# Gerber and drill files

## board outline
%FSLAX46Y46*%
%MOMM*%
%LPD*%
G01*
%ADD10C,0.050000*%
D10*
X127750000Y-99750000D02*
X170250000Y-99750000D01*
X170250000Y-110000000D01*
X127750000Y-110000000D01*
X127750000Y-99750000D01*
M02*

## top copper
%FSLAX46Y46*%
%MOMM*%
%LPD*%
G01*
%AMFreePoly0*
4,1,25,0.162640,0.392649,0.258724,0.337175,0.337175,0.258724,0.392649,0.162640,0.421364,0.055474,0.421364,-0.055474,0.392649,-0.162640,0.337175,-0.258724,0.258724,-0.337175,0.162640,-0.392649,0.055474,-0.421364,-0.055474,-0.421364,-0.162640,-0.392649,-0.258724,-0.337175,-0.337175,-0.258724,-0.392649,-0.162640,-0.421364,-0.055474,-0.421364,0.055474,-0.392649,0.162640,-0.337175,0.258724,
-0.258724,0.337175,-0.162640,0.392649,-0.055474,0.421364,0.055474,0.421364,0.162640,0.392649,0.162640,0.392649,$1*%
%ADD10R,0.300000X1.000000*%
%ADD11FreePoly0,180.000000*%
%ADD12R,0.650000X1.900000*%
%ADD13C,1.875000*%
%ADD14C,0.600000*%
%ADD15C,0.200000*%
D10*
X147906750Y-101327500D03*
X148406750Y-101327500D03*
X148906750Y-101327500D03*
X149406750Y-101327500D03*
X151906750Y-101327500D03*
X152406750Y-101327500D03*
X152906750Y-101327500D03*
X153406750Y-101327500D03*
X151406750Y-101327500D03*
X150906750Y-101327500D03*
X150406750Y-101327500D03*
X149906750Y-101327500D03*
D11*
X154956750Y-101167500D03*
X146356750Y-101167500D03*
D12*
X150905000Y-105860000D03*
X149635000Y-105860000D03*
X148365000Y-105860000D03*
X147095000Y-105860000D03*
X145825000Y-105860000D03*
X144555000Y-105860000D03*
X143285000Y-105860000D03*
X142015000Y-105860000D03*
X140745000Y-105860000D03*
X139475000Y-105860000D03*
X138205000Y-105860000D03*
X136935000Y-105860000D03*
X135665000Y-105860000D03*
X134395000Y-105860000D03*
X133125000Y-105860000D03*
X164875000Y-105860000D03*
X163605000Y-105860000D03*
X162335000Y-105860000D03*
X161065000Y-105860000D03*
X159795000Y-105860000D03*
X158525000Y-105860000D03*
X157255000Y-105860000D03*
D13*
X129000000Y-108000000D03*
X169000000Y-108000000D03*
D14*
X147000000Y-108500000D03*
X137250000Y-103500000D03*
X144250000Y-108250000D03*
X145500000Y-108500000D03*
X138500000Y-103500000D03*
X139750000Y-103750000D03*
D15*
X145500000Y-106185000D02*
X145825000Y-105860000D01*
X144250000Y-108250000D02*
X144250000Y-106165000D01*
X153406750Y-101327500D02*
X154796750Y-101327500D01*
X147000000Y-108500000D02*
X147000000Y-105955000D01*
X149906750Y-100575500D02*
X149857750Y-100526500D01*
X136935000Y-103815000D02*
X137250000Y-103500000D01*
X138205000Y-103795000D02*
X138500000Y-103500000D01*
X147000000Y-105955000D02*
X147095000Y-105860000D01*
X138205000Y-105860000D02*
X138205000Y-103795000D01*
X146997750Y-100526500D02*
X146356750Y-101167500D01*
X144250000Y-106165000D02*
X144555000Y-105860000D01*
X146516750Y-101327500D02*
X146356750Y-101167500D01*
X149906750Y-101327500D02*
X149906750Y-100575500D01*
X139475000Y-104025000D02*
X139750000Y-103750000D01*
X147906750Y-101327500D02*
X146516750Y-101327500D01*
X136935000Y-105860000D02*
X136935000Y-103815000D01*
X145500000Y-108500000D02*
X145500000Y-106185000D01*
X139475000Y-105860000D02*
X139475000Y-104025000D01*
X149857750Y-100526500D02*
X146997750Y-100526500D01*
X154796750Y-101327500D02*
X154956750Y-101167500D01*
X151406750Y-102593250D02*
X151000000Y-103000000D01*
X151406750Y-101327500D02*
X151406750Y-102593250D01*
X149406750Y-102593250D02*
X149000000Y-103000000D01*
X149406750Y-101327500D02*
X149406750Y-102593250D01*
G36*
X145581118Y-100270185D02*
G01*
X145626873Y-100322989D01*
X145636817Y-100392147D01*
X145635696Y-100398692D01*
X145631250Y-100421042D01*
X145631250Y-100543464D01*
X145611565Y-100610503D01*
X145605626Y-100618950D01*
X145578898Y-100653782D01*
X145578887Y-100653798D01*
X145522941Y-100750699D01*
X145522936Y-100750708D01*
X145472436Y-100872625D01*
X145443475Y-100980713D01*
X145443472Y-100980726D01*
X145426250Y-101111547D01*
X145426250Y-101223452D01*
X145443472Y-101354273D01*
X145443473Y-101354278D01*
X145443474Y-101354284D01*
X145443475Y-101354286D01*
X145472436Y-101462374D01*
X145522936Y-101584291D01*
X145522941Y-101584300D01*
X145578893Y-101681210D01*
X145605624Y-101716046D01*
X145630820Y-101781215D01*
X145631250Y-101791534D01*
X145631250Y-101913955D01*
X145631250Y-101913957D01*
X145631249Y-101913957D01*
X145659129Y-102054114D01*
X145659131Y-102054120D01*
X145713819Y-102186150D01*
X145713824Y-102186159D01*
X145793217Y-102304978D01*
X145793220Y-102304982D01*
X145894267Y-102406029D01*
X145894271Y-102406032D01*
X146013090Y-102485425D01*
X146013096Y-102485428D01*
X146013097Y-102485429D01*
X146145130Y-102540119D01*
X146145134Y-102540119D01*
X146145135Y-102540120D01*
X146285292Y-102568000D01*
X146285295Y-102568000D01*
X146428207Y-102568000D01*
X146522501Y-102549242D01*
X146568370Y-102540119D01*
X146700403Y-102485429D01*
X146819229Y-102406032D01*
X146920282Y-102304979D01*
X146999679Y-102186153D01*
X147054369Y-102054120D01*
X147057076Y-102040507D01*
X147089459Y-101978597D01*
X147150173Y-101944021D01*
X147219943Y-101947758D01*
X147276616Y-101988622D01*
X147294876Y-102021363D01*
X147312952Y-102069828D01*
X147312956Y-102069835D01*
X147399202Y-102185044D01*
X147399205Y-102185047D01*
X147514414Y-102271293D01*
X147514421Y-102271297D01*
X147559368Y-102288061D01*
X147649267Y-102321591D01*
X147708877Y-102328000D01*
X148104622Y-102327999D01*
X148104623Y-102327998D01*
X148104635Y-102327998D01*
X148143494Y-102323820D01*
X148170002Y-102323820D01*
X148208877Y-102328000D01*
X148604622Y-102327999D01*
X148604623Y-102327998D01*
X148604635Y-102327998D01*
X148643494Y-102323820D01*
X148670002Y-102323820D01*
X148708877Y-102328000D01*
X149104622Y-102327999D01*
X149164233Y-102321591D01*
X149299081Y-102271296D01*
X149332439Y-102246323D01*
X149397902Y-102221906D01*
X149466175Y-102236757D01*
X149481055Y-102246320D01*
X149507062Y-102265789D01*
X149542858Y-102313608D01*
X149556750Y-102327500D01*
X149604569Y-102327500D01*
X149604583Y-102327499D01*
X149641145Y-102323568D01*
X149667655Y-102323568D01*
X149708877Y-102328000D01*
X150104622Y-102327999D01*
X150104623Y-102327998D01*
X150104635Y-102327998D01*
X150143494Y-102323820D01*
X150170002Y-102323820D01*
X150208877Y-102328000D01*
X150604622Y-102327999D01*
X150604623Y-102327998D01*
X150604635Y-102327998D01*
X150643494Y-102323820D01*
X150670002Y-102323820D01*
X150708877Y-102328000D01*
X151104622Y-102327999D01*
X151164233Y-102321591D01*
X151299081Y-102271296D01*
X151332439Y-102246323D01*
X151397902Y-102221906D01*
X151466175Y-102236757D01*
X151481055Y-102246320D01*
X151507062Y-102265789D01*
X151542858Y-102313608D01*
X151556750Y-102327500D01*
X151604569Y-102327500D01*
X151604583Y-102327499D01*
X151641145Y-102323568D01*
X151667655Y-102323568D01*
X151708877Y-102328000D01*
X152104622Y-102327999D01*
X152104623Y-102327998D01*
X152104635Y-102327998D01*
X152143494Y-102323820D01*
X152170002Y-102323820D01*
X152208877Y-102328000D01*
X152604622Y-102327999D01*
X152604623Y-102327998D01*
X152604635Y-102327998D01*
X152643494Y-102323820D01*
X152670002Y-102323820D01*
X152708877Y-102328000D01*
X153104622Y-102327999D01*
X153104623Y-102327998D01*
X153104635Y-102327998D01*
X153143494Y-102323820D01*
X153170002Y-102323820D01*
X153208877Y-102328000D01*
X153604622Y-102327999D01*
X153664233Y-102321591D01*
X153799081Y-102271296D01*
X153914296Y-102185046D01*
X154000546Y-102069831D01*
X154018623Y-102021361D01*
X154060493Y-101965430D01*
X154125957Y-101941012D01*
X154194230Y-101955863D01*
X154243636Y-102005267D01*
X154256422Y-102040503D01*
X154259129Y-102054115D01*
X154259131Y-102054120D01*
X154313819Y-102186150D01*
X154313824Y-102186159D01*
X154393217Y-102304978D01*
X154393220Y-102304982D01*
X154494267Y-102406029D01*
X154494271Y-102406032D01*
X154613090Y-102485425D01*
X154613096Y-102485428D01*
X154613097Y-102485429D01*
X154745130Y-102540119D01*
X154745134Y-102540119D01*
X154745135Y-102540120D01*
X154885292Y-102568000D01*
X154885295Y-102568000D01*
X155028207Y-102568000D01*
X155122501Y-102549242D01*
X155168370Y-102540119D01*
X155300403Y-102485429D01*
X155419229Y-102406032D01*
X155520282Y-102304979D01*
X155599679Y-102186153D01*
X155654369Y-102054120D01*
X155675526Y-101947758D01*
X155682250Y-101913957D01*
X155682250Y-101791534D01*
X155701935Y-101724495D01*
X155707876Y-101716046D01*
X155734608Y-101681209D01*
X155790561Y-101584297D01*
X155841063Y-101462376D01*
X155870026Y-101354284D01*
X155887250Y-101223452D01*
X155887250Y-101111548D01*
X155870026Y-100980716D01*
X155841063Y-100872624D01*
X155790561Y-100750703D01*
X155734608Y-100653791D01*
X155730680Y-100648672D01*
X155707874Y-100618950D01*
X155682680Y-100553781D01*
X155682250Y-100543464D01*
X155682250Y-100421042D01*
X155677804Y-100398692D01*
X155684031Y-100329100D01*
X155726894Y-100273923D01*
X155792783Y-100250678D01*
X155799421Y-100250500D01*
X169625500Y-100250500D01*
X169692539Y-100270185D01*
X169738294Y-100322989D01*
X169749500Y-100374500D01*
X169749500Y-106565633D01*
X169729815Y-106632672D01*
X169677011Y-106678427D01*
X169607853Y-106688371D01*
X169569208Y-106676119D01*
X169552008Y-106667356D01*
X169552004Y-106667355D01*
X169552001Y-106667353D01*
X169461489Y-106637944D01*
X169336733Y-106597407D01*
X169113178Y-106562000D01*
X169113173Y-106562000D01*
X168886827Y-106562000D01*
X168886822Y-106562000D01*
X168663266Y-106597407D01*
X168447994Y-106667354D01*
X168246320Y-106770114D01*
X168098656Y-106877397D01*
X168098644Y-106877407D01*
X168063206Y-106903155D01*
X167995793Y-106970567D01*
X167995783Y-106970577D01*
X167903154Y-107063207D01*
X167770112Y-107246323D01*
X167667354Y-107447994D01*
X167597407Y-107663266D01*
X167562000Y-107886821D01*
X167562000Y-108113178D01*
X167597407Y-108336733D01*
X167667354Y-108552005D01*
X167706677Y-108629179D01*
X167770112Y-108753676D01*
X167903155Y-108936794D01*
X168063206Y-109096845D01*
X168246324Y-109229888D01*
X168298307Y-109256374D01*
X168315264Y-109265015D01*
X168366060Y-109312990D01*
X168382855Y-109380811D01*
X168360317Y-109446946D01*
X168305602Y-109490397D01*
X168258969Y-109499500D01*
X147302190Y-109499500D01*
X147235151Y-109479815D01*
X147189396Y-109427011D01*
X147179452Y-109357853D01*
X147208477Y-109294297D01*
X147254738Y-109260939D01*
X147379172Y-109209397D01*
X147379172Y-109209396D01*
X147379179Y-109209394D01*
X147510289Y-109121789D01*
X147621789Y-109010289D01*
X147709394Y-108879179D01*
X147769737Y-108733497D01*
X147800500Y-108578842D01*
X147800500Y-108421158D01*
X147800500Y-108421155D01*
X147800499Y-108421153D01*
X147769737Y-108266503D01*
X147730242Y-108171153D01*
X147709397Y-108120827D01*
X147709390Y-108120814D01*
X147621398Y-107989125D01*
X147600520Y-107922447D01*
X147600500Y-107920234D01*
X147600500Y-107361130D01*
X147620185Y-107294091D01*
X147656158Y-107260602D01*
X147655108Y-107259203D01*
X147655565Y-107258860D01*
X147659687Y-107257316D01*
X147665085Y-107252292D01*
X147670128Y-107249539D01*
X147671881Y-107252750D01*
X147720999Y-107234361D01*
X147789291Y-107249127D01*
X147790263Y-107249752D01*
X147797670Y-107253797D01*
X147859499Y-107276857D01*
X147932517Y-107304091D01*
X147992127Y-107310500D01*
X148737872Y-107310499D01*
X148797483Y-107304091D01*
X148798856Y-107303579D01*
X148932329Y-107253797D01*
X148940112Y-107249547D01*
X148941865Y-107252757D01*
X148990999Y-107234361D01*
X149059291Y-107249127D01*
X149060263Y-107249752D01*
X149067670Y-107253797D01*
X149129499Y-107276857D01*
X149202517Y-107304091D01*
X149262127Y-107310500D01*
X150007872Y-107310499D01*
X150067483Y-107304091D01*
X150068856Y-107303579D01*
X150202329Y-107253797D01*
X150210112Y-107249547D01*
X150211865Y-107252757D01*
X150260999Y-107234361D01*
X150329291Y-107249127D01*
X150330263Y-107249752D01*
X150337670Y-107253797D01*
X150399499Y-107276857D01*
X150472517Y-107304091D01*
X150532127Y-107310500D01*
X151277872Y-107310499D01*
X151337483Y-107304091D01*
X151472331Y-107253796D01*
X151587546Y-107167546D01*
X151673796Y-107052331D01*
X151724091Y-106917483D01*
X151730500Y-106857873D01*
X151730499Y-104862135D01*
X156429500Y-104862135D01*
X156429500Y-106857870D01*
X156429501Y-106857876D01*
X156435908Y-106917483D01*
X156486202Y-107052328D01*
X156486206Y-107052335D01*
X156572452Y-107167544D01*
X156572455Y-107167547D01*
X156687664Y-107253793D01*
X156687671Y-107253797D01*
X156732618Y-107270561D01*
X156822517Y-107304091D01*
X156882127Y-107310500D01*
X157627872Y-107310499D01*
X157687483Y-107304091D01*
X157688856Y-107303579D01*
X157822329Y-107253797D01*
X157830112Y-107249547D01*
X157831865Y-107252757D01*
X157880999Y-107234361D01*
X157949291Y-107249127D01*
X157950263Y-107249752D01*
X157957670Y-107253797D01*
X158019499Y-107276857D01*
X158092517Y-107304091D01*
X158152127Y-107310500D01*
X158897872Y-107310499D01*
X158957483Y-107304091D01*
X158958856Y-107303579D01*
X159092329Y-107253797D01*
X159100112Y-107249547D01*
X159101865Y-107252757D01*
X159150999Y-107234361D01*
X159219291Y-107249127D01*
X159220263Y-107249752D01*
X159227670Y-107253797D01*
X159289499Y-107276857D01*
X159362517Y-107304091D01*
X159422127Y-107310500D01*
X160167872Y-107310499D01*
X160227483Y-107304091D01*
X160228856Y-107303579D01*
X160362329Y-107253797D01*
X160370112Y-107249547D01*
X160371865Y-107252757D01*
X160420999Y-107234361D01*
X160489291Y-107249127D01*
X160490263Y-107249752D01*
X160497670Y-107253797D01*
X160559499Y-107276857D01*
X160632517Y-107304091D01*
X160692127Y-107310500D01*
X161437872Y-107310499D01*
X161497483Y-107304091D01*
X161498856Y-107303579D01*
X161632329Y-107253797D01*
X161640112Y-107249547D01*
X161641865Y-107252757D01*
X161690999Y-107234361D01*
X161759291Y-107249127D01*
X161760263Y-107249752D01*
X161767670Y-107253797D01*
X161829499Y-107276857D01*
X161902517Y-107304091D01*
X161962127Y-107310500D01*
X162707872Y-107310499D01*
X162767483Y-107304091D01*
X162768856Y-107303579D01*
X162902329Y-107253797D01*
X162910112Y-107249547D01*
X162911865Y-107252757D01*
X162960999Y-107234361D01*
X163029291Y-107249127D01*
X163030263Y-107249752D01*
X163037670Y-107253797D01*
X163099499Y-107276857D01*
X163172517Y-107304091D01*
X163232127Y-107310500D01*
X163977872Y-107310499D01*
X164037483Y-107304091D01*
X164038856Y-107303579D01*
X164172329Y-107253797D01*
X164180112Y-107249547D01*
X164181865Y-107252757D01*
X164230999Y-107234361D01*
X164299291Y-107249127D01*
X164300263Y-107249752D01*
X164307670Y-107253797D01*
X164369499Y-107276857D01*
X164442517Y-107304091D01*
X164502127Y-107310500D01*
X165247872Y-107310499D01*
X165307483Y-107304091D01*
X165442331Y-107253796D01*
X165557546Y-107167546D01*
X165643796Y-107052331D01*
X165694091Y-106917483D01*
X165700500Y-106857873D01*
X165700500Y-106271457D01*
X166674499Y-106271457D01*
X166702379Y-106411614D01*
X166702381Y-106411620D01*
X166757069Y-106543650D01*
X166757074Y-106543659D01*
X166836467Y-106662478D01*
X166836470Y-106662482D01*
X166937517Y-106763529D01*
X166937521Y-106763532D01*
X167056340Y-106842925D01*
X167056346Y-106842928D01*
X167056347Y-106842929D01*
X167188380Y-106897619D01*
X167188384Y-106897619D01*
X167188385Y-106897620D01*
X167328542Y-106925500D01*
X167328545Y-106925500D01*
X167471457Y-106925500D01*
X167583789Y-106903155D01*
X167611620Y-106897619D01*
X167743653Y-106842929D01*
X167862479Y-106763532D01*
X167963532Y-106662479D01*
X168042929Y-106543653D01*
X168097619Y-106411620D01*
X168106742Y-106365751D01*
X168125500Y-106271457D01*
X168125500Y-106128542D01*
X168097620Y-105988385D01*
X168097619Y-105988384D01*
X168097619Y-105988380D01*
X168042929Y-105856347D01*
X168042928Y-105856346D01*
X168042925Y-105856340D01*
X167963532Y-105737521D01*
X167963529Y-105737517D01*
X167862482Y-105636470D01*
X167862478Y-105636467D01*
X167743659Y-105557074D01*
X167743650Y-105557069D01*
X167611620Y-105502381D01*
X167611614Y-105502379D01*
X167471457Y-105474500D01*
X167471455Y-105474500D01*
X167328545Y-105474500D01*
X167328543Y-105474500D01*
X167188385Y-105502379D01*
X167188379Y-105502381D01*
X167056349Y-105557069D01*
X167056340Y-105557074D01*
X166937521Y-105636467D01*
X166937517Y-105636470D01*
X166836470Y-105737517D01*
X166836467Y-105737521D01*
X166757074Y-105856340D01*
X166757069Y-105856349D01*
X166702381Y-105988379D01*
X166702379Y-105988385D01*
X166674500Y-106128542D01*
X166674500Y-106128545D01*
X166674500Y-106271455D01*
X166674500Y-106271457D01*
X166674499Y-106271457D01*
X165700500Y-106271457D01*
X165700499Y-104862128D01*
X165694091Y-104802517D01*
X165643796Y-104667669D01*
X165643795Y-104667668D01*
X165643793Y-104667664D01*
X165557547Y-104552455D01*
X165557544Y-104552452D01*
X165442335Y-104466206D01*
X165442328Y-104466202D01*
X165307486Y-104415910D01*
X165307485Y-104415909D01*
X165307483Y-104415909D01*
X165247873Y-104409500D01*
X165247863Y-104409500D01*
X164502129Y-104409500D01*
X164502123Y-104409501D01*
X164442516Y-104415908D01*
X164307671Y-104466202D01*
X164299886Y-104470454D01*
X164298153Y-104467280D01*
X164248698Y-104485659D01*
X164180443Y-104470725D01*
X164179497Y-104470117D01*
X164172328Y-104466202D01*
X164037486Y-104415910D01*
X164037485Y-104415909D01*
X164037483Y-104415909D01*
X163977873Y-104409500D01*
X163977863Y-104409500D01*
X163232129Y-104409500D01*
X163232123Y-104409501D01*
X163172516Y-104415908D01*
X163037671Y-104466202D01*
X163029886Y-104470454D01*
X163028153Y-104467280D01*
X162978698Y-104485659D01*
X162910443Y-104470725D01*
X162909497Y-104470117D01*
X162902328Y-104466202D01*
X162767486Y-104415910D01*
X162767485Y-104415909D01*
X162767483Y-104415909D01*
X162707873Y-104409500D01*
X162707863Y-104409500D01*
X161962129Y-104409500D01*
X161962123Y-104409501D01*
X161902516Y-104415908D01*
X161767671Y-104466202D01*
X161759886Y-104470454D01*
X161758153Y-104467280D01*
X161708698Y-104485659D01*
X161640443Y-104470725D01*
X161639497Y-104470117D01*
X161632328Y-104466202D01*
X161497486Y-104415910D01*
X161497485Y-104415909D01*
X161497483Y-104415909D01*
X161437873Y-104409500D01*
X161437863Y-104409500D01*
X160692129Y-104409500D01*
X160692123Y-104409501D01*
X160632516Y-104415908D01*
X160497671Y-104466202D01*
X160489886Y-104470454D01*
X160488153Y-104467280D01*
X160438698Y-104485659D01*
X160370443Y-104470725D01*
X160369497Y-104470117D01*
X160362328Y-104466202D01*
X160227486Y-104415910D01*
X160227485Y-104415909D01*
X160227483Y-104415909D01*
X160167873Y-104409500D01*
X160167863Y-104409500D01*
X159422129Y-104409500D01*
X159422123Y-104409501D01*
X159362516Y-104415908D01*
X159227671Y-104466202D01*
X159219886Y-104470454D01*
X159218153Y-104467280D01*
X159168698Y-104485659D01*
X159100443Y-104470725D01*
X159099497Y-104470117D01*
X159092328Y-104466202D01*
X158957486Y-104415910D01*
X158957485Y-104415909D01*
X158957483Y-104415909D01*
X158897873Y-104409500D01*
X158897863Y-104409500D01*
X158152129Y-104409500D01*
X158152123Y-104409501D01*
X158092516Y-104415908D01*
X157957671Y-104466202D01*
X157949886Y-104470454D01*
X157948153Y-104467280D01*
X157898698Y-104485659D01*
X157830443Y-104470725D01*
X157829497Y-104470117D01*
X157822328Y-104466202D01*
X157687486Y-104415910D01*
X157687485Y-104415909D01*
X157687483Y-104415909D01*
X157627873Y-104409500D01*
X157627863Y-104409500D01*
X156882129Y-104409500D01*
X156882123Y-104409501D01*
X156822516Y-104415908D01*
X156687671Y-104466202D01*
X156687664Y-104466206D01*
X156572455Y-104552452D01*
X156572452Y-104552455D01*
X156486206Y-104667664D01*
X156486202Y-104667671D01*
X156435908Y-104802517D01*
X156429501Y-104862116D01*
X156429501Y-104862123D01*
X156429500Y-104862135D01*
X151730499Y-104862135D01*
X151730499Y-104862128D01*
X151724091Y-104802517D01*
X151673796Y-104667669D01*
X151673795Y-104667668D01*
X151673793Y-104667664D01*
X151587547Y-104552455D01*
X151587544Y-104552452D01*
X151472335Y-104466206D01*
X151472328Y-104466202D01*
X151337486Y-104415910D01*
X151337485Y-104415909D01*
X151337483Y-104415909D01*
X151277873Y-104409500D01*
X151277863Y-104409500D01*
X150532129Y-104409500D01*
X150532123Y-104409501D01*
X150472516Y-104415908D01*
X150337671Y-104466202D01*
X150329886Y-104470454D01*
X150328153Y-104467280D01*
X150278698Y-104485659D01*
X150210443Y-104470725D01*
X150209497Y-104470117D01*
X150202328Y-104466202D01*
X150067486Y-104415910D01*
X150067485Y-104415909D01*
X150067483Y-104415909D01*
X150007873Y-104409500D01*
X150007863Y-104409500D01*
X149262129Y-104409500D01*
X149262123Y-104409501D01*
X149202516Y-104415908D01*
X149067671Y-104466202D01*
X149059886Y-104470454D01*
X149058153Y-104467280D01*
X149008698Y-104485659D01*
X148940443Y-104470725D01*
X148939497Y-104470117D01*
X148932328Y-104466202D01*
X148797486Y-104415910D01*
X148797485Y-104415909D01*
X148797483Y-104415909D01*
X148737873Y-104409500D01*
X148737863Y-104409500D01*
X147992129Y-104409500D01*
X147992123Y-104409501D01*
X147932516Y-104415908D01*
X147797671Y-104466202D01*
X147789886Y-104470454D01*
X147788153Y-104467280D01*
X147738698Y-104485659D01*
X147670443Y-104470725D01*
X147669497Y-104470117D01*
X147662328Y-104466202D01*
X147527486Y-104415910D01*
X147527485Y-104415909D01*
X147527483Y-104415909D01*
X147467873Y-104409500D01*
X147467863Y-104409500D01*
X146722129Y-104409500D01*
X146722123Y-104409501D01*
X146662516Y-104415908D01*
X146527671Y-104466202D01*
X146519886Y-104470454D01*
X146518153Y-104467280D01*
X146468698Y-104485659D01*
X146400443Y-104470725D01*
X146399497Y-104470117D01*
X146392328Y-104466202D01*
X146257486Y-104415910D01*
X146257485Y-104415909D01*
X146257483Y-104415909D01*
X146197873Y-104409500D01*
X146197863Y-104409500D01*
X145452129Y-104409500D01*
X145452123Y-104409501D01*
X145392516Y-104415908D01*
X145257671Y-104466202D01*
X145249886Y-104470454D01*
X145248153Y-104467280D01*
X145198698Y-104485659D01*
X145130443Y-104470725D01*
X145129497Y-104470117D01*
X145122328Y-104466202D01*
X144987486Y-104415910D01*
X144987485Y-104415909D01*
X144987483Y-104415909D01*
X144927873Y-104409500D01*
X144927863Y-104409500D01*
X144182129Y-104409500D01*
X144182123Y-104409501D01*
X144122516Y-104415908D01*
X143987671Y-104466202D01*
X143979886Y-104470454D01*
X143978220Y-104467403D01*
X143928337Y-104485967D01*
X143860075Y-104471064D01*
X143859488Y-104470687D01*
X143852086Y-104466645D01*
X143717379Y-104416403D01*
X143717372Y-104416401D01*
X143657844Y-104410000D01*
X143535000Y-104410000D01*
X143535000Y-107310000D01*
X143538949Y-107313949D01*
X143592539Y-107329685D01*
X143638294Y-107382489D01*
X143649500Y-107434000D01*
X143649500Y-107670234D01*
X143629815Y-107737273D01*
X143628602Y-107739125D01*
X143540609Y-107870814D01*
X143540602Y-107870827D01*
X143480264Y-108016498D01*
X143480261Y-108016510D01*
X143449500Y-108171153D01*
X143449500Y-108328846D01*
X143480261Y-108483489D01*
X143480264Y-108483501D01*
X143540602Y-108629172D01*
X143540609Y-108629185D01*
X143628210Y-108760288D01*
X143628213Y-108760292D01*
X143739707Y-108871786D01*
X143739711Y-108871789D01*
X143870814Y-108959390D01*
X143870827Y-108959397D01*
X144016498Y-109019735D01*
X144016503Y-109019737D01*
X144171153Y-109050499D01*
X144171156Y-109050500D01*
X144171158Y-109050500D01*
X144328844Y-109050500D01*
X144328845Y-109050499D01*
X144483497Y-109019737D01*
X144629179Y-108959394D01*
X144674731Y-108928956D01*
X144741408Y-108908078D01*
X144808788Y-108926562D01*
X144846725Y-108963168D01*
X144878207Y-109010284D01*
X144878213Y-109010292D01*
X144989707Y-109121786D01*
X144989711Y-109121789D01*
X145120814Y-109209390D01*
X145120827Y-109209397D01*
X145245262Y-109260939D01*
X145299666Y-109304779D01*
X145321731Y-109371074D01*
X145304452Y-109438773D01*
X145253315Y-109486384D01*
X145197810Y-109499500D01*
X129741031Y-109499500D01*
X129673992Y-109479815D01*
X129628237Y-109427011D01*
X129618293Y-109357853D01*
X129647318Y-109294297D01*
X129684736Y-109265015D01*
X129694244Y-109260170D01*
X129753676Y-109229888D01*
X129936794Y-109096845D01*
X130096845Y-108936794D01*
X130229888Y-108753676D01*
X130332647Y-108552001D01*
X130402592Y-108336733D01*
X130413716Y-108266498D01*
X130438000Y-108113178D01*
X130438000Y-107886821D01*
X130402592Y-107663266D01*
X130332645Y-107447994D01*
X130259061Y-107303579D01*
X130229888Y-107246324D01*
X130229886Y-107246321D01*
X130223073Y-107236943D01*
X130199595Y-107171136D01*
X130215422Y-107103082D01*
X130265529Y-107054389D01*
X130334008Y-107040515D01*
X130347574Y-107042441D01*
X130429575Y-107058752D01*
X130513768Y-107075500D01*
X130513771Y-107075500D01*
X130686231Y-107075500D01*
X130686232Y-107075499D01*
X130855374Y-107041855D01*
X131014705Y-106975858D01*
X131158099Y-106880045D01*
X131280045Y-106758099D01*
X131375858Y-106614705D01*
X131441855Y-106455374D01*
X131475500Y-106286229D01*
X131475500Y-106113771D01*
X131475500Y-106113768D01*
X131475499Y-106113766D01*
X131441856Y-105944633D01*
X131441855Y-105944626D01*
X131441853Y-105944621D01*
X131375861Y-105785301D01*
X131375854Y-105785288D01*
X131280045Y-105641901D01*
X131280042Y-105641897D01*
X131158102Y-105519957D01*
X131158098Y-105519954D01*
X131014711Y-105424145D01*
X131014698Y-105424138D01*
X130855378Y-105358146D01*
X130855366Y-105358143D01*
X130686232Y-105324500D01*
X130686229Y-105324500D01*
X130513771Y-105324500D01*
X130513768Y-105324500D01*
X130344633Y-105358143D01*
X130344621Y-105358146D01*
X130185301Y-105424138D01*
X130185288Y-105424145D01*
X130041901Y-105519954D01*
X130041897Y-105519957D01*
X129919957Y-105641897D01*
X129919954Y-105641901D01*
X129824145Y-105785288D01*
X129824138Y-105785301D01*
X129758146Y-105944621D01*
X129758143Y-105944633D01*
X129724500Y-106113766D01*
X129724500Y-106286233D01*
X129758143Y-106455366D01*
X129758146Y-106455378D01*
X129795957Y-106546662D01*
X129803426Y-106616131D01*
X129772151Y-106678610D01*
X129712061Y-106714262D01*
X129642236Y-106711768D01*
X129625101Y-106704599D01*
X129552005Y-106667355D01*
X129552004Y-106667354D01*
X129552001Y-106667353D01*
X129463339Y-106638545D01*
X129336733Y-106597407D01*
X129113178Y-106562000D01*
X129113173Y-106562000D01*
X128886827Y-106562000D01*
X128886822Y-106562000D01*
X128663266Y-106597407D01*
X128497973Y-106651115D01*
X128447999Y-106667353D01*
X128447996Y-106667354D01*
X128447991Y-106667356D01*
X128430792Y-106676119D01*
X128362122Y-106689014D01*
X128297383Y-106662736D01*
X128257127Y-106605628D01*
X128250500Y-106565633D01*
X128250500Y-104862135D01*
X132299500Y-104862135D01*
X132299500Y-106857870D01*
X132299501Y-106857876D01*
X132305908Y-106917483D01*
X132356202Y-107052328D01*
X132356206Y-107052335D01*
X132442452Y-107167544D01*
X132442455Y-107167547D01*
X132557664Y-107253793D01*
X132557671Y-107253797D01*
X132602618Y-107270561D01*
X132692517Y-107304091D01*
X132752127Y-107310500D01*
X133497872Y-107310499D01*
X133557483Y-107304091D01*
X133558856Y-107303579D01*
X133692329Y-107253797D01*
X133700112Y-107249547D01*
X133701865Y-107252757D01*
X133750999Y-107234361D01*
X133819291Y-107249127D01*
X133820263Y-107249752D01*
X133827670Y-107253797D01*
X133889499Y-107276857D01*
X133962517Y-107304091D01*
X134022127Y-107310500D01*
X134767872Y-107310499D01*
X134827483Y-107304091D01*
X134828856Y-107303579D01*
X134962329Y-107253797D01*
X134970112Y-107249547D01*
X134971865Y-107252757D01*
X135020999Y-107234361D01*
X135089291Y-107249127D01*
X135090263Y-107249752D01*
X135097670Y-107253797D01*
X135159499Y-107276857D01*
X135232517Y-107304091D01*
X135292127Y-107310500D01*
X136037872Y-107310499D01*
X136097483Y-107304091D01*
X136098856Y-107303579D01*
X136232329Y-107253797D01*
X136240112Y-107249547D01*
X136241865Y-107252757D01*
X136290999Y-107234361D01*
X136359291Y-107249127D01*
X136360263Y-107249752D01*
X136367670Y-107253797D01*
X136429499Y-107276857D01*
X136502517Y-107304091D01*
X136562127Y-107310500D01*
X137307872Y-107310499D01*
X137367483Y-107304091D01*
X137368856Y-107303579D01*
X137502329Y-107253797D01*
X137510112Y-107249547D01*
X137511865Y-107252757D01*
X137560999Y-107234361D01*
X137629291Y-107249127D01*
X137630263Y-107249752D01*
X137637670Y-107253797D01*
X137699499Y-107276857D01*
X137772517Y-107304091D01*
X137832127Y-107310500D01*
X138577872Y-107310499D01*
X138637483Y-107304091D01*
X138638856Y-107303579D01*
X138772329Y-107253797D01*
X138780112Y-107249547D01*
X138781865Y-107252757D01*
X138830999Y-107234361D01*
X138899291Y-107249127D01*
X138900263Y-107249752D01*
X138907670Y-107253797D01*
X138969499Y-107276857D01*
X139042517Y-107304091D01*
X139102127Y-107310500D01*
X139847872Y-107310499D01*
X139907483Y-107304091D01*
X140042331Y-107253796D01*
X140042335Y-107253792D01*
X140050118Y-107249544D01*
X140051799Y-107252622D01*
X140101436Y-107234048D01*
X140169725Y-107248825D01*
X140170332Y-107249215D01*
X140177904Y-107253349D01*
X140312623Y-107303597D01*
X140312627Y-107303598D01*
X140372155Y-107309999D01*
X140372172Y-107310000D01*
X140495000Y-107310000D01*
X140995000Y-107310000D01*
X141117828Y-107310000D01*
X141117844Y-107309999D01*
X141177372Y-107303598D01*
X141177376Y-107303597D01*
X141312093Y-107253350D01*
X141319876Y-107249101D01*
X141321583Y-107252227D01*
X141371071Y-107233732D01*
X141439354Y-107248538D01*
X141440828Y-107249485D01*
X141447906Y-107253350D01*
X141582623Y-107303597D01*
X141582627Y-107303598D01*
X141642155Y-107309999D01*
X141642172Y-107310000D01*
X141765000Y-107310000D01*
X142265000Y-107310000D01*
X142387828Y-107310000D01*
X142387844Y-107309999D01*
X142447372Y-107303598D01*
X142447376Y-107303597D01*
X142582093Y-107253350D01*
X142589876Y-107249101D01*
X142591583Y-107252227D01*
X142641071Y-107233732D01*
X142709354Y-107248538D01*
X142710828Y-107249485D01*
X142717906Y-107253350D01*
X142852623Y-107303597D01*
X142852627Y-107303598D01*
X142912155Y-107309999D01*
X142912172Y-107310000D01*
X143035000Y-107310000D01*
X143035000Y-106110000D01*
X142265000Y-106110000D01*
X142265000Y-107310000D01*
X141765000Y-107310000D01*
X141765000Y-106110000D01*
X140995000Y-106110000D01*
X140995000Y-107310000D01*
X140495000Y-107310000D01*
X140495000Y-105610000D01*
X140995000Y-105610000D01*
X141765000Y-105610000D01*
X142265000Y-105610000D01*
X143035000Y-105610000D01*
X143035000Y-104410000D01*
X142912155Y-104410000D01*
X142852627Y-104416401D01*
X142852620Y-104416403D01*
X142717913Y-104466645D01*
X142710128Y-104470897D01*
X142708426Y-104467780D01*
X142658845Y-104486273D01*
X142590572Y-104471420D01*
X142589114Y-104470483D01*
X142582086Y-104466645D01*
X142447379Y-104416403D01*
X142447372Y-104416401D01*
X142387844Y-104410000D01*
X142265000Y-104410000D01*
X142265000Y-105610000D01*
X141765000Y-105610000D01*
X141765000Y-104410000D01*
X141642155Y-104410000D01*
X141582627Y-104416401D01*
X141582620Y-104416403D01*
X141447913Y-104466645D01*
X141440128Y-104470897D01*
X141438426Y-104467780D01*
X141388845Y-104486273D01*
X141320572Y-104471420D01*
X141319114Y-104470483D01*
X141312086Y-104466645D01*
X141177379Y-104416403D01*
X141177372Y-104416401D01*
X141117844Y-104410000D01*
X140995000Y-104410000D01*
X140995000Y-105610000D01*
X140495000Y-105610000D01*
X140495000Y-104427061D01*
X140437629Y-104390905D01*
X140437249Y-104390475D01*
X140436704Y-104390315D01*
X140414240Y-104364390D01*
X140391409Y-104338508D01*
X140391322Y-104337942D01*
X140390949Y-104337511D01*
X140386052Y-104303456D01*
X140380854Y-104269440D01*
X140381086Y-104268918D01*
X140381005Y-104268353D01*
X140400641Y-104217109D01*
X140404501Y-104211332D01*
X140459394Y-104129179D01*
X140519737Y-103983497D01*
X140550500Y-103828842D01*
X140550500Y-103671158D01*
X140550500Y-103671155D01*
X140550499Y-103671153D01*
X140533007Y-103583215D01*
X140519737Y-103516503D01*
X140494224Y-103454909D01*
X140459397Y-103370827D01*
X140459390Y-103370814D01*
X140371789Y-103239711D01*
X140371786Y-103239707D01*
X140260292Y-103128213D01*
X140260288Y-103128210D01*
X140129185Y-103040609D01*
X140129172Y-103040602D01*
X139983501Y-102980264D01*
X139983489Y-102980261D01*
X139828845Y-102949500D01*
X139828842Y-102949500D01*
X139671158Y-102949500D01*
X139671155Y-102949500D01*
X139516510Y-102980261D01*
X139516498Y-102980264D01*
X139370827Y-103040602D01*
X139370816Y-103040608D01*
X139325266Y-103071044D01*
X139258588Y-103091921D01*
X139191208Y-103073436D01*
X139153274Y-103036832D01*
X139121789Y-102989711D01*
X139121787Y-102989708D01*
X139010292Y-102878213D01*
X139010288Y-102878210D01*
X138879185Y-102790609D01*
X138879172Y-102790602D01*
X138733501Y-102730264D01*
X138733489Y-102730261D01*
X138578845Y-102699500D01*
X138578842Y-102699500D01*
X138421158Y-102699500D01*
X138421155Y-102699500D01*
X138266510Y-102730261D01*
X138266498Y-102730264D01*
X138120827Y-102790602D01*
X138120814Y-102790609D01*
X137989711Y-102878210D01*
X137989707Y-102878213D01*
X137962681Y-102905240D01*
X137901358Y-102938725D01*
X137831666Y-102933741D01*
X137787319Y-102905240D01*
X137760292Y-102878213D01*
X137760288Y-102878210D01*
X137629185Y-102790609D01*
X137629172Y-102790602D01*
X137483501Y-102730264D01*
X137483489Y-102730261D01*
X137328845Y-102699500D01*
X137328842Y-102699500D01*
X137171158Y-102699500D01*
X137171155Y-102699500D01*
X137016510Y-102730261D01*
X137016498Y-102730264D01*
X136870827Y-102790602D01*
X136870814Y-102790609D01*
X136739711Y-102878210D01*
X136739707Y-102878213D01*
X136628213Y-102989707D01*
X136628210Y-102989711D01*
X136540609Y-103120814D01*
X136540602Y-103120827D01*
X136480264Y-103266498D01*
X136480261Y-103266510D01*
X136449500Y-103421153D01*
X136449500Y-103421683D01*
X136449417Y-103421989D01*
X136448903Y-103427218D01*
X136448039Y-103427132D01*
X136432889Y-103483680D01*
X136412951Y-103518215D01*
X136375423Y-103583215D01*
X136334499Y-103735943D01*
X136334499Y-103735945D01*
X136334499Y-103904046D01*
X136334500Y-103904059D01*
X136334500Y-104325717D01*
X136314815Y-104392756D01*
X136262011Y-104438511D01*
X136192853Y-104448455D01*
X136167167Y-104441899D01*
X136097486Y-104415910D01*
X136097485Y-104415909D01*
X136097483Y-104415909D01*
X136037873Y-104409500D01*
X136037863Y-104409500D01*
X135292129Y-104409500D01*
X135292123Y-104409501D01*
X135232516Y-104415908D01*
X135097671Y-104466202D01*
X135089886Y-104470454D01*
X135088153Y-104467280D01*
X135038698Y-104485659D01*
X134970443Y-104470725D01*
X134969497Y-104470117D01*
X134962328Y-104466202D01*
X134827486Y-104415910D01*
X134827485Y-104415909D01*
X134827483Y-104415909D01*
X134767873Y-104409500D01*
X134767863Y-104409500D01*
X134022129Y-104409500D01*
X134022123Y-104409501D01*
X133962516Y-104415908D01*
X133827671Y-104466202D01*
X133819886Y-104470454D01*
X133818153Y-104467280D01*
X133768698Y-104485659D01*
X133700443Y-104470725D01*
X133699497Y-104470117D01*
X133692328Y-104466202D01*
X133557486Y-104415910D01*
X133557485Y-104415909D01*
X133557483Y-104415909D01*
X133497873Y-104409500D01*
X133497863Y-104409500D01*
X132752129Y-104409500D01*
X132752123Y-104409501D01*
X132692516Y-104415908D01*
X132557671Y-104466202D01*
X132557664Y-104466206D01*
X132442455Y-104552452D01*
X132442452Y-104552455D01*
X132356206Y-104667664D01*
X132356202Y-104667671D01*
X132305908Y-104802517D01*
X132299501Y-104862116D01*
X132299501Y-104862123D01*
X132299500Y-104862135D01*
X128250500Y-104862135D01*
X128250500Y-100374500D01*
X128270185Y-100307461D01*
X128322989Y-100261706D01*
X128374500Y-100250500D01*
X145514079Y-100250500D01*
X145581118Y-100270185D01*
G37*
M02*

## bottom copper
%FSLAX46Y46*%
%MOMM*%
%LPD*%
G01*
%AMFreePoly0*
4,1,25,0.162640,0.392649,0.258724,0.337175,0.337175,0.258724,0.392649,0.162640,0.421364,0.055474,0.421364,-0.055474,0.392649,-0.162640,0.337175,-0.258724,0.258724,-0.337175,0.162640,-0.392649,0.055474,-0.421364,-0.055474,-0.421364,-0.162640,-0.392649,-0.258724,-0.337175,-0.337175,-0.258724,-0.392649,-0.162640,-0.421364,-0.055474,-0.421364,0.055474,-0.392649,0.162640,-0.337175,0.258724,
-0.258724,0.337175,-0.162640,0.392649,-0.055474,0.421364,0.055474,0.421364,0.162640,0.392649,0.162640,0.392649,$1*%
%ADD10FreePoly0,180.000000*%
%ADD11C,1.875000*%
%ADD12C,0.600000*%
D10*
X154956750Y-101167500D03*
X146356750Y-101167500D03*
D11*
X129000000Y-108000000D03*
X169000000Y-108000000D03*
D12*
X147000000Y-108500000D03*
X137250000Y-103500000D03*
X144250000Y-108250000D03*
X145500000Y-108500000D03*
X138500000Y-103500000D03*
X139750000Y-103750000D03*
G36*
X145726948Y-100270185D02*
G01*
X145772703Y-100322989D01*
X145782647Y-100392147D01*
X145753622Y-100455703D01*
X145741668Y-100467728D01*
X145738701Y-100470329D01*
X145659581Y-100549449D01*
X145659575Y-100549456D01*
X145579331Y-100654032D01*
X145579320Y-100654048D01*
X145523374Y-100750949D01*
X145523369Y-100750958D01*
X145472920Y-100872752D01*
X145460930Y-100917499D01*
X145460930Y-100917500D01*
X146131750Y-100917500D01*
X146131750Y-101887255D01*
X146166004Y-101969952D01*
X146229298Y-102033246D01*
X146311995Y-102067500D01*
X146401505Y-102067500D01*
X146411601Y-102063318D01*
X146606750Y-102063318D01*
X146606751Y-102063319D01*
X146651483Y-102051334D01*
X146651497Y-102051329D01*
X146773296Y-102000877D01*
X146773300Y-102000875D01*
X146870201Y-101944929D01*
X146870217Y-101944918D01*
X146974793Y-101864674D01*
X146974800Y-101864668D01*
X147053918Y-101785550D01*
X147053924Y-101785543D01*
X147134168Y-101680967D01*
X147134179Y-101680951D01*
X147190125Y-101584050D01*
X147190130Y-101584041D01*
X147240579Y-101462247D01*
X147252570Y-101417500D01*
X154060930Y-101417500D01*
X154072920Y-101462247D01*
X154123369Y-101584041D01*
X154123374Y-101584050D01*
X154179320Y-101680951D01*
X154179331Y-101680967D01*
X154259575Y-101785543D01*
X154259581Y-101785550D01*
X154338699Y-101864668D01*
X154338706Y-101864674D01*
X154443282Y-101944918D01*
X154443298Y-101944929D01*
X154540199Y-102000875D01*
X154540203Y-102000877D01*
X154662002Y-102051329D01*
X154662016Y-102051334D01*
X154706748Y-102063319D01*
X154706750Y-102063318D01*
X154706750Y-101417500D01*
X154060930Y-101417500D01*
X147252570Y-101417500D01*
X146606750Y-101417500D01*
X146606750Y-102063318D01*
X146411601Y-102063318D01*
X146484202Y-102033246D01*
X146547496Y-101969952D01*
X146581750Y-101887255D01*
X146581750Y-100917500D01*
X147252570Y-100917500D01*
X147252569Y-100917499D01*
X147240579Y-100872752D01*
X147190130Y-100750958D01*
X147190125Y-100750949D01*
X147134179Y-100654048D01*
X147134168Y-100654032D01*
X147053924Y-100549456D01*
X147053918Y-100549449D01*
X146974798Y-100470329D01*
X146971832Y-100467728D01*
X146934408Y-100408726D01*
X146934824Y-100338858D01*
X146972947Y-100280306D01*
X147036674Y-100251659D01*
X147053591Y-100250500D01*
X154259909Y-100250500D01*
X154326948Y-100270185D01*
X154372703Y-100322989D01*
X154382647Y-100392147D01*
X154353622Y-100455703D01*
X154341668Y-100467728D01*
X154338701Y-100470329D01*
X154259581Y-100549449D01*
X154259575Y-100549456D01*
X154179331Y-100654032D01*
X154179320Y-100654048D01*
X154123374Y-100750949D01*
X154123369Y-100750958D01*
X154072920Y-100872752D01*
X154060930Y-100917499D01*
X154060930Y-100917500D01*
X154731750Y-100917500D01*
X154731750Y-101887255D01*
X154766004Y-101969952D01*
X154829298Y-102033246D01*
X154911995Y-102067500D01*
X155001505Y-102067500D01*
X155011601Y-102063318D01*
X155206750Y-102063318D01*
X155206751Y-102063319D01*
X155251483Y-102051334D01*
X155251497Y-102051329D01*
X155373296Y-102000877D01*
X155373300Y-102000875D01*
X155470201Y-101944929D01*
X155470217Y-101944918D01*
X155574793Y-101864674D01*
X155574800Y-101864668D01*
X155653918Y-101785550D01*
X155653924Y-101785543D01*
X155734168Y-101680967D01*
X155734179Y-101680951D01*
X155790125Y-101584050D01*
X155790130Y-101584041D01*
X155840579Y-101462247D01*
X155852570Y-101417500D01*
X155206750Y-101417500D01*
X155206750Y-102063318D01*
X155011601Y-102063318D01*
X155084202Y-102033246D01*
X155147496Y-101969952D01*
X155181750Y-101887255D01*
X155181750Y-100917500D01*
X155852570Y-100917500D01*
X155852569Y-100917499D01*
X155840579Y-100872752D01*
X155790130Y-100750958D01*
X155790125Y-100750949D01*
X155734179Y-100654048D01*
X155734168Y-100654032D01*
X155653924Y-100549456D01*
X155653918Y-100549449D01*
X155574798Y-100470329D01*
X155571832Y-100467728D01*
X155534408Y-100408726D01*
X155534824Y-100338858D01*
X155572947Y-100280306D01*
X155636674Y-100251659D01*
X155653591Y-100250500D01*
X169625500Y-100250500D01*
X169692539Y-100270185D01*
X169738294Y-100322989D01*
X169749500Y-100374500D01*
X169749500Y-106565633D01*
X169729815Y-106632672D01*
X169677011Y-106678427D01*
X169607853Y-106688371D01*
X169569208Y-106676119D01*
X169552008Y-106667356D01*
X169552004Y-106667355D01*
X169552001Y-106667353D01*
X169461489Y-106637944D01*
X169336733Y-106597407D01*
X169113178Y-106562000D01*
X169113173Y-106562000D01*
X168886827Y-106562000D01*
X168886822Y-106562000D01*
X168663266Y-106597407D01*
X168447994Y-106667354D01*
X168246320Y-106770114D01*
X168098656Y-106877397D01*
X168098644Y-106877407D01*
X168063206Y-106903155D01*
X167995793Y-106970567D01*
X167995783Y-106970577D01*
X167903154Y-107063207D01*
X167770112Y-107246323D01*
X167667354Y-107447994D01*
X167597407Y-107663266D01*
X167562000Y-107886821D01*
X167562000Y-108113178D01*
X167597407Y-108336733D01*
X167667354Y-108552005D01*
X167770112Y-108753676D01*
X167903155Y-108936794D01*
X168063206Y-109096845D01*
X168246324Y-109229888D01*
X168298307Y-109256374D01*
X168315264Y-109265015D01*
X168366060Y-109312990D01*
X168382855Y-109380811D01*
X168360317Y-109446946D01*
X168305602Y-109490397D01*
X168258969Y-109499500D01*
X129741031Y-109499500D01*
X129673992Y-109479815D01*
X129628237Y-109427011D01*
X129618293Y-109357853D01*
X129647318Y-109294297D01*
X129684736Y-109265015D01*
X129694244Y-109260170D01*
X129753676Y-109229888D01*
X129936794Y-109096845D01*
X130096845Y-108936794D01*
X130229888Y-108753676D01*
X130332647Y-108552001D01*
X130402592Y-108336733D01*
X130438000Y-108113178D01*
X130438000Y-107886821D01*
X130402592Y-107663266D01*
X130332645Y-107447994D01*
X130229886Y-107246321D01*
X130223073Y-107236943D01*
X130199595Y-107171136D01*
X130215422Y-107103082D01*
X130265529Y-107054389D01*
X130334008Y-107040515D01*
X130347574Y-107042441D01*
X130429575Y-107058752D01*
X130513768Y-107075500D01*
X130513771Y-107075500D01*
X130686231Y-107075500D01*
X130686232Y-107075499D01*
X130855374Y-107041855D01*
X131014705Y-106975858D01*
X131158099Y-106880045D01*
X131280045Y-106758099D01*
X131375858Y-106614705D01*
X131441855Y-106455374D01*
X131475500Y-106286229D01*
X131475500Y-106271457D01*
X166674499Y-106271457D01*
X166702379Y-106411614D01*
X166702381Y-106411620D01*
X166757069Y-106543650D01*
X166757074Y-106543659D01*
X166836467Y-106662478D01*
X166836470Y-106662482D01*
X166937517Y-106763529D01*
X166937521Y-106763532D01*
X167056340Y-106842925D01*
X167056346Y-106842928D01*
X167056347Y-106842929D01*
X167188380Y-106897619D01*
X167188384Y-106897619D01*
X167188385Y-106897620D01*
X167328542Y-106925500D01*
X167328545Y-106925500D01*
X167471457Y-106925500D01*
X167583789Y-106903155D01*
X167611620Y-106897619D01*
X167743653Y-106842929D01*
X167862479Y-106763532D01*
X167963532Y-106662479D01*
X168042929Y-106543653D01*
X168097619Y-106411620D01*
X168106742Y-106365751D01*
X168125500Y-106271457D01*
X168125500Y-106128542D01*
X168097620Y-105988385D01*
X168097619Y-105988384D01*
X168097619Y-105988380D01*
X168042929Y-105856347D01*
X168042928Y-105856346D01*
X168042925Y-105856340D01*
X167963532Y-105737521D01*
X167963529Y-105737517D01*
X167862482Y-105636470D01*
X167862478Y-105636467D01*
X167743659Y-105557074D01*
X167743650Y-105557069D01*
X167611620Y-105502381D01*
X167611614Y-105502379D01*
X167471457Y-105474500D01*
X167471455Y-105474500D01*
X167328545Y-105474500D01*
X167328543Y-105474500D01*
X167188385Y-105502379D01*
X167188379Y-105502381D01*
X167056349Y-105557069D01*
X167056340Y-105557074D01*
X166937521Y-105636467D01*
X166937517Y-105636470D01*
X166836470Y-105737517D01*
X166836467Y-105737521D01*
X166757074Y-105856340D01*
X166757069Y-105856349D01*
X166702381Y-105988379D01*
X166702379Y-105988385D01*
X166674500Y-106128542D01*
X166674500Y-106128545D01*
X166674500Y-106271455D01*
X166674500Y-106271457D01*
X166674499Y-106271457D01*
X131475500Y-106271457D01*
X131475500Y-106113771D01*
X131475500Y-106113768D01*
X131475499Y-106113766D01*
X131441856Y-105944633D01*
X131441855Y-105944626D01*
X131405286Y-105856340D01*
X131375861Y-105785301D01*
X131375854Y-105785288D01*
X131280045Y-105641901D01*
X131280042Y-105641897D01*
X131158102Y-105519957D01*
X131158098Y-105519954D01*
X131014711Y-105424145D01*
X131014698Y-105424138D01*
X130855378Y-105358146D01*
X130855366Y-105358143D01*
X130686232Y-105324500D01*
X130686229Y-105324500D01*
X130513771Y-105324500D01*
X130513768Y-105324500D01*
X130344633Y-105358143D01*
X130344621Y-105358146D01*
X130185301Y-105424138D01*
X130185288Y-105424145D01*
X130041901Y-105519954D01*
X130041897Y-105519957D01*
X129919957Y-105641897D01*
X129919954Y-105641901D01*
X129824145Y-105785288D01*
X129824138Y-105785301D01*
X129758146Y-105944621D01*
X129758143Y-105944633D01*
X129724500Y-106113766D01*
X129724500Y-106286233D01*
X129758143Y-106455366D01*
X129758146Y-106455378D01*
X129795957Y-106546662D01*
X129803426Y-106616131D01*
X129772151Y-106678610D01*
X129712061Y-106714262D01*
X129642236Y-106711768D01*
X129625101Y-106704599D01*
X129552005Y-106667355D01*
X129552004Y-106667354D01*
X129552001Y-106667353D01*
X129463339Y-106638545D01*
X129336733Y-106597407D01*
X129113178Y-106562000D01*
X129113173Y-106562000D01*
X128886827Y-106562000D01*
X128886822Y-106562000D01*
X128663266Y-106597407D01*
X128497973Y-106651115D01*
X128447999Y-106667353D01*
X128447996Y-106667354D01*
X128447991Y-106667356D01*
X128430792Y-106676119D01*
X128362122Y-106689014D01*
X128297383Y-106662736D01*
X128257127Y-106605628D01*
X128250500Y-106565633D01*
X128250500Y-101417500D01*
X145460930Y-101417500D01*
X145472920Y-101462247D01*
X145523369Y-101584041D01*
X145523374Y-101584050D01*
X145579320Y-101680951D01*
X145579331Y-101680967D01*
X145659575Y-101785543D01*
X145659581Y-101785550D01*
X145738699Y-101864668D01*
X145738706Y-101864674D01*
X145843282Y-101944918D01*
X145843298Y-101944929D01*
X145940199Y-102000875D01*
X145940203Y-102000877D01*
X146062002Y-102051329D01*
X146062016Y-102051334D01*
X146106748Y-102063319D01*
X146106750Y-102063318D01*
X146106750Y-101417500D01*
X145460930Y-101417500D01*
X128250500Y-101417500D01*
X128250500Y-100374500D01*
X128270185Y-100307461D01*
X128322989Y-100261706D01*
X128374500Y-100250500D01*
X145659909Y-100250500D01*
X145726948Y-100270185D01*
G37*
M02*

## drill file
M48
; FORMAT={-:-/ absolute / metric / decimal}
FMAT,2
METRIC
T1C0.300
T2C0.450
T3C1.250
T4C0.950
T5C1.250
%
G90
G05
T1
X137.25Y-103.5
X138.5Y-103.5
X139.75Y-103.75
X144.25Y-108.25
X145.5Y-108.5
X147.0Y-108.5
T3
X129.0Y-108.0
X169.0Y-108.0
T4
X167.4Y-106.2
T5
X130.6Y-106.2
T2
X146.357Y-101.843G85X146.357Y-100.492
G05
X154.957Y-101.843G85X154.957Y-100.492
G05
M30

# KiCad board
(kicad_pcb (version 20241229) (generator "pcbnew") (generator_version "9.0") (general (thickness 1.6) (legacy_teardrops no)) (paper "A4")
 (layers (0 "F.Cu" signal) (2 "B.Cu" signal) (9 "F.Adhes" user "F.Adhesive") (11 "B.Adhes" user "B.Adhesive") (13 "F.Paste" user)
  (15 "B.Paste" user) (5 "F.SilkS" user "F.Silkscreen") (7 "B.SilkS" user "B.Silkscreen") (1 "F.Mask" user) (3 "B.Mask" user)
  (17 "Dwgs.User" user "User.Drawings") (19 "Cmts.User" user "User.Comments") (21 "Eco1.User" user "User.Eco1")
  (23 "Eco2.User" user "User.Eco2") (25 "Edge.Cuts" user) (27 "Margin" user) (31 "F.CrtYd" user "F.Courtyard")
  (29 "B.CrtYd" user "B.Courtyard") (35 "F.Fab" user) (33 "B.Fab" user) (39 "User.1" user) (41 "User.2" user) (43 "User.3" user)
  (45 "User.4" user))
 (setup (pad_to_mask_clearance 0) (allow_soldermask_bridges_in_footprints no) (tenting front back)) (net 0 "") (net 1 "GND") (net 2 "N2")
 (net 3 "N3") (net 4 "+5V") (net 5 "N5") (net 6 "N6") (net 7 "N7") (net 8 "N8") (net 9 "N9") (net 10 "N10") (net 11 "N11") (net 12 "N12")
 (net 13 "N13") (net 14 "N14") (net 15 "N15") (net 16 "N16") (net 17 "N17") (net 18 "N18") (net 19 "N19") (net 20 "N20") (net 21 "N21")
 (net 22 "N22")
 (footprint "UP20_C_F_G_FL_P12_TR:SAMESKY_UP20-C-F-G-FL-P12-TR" (layer "F.Cu") (at 150.65675 99.7675 180)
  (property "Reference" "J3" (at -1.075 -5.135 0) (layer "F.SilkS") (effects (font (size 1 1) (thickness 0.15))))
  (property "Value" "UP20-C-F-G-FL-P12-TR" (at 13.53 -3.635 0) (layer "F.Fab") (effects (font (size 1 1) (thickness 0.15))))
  (pad "A1" smd rect (at 2.75 -1.56 180) (size 0.3 1) (layers "F.Cu" "F.Mask" "F.Paste") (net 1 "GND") (solder_mask_margin 0.102))
  (pad "A2" smd rect (at 2.25 -1.56 180) (size 0.3 1) (layers "F.Cu" "F.Mask" "F.Paste") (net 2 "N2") (solder_mask_margin 0.102))
  (pad "A3" smd rect (at 1.75 -1.56 180) (size 0.3 1) (layers "F.Cu" "F.Mask" "F.Paste") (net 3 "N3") (solder_mask_margin 0.102))
  (pad "A4" smd rect (at 1.25 -1.56 180) (size 0.3 1) (layers "F.Cu" "F.Mask" "F.Paste") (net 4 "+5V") (solder_mask_margin 0.102))
  (pad "A5" smd rect (at -1.25 -1.56 180) (size 0.3 1) (layers "F.Cu" "F.Mask" "F.Paste") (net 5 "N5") (solder_mask_margin 0.102))
  (pad "A6" smd rect (at -1.75 -1.56 180) (size 0.3 1) (layers "F.Cu" "F.Mask" "F.Paste") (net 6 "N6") (solder_mask_margin 0.102))
  (pad "A7" smd rect (at -2.25 -1.56 180) (size 0.3 1) (layers "F.Cu" "F.Mask" "F.Paste") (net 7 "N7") (solder_mask_margin 0.102))
  (pad "A12" smd rect (at -2.75 -1.56 180) (size 0.3 1) (layers "F.Cu" "F.Mask" "F.Paste") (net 1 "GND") (solder_mask_margin 0.102))
  (pad "B9" smd rect (at -0.75 -1.56 180) (size 0.3 1) (layers "F.Cu" "F.Mask" "F.Paste") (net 4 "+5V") (solder_mask_margin 0.102))
  (pad "B10" smd rect (at -0.25 -1.56 180) (size 0.3 1) (layers "F.Cu" "F.Mask" "F.Paste") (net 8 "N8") (solder_mask_margin 0.102))
  (pad "B11" smd rect (at 0.25 -1.56 180) (size 0.3 1) (layers "F.Cu" "F.Mask" "F.Paste") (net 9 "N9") (solder_mask_margin 0.102))
  (pad "B12" smd rect (at 0.75 -1.56 180) (size 0.3 1) (layers "F.Cu" "F.Mask" "F.Paste") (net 1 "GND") (solder_mask_margin 0.102))
  (pad "SH1" thru_hole custom (at -4.3 -1.4 180) (size 0.85 2.25) (drill oval 0.45 1.8) (layers "*.Cu") (remove_unused_layers no)
   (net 1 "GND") (thermal_bridge_angle 90) (options (clearance outline) (anchor circle)) (primitives))
  (pad "SH2" thru_hole custom (at 4.3 -1.4 180) (size 0.85 2.25) (drill oval 0.45 1.8) (layers "*.Cu") (remove_unused_layers no)
   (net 1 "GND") (thermal_bridge_angle 90) (options (clearance outline) (anchor circle)) (primitives)))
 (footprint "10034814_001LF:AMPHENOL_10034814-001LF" (layer "F.Cu") (at 149 108)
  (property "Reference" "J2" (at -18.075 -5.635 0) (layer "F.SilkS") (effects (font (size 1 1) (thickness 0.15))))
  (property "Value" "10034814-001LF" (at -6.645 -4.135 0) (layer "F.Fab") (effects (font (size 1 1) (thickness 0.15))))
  (pad "" np_thru_hole circle (at -18.4 -1.8) (size 1.25 1.25) (drill 1.25) (layers "*.Cu" "*.Mask"))
  (pad "" np_thru_hole circle (at 18.4 -1.8) (size 0.95 0.95) (drill 0.95) (layers "*.Cu" "*.Mask"))
  (pad "P1" smd rect (at 1.905 -2.14) (size 0.65 1.9) (layers "F.Cu" "F.Mask" "F.Paste") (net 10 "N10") (solder_mask_margin 0.102))
  (pad "P2" smd rect (at 0.635 -2.14) (size 0.65 1.9) (layers "F.Cu" "F.Mask" "F.Paste") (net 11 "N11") (solder_mask_margin 0.102))
  (pad "P3" smd rect (at -0.635 -2.14) (size 0.65 1.9) (layers "F.Cu" "F.Mask" "F.Paste") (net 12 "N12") (solder_mask_margin 0.102))
  (pad "P4" smd rect (at -1.905 -2.14) (size 0.65 1.9) (layers "F.Cu" "F.Mask" "F.Paste") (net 1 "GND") (solder_mask_margin 0.102))
  (pad "P5" smd rect (at -3.175 -2.14) (size 0.65 1.9) (layers "F.Cu" "F.Mask" "F.Paste") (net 1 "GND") (solder_mask_margin 0.102))
  (pad "P6" smd rect (at -4.445 -2.14) (size 0.65 1.9) (layers "F.Cu" "F.Mask" "F.Paste") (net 1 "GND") (solder_mask_margin 0.102))
  (pad "P7" smd rect (at -5.715 -2.14) (size 0.65 1.9) (layers "F.Cu" "F.Mask" "F.Paste") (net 4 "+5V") (solder_mask_margin 0.102))
  (pad "P8" smd rect (at -6.985 -2.14) (size 0.65 1.9) (layers "F.Cu" "F.Mask" "F.Paste") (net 4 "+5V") (solder_mask_margin 0.102))
  (pad "P9" smd rect (at -8.255 -2.14) (size 0.65 1.9) (layers "F.Cu" "F.Mask" "F.Paste") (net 4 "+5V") (solder_mask_margin 0.102))
  (pad "P10" smd rect (at -9.525 -2.14) (size 0.65 1.9) (layers "F.Cu" "F.Mask" "F.Paste") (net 1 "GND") (solder_mask_margin 0.102))
  (pad "P11" smd rect (at -10.795 -2.14) (size 0.65 1.9) (layers "F.Cu" "F.Mask" "F.Paste") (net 1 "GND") (solder_mask_margin 0.102))
  (pad "P12" smd rect (at -12.065 -2.14) (size 0.65 1.9) (layers "F.Cu" "F.Mask" "F.Paste") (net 1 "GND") (solder_mask_margin 0.102))
  (pad "P13" smd rect (at -13.335 -2.14) (size 0.65 1.9) (layers "F.Cu" "F.Mask" "F.Paste") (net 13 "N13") (solder_mask_margin 0.102))
  (pad "P14" smd rect (at -14.605 -2.14) (size 0.65 1.9) (layers "F.Cu" "F.Mask" "F.Paste") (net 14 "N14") (solder_mask_margin 0.102))
  (pad "P15" smd rect (at -15.875 -2.14) (size 0.65 1.9) (layers "F.Cu" "F.Mask" "F.Paste") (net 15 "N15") (solder_mask_margin 0.102))
  (pad "S1" smd rect (at 15.875 -2.14) (size 0.65 1.9) (layers "F.Cu" "F.Mask" "F.Paste") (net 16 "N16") (solder_mask_margin 0.102))
  (pad "S2" smd rect (at 14.605 -2.14) (size 0.65 1.9) (layers "F.Cu" "F.Mask" "F.Paste") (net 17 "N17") (solder_mask_margin 0.102))
  (pad "S3" smd rect (at 13.335 -2.14) (size 0.65 1.9) (layers "F.Cu" "F.Mask" "F.Paste") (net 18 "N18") (solder_mask_margin 0.102))
  (pad "S4" smd rect (at 12.065 -2.14) (size 0.65 1.9) (layers "F.Cu" "F.Mask" "F.Paste") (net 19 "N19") (solder_mask_margin 0.102))
  (pad "S5" smd rect (at 10.795 -2.14) (size 0.65 1.9) (layers "F.Cu" "F.Mask" "F.Paste") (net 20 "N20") (solder_mask_margin 0.102))
  (pad "S6" smd rect (at 9.525 -2.14) (size 0.65 1.9) (layers "F.Cu" "F.Mask" "F.Paste") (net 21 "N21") (solder_mask_margin 0.102))
  (pad "S7" smd rect (at 8.255 -2.14) (size 0.65 1.9) (layers "F.Cu" "F.Mask" "F.Paste") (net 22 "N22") (solder_mask_margin 0.102))
  (pad "SH1" thru_hole circle (at -20 0) (size 1.875 1.875) (drill 1.25) (layers "*.Cu" "*.Mask") (remove_unused_layers no)
   (solder_mask_margin 0.102))
  (pad "SH2" thru_hole circle (at 20 0) (size 1.875 1.875) (drill 1.25) (layers "*.Cu" "*.Mask") (remove_unused_layers no)
   (solder_mask_margin 0.102)))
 (gr_rect (start 127.75 99.75) (end 170.25 110) (stroke (width 0.05) (type default)) (fill no) (layer "Edge.Cuts"))
 (segment (start 145.5 106.185) (end 145.825 105.86) (width 0.2) (layer "F.Cu") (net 1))
 (segment (start 144.25 108.25) (end 144.25 106.165) (width 0.2) (layer "F.Cu") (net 1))
 (segment (start 153.40675 101.3275) (end 154.79675 101.3275) (width 0.2) (layer "F.Cu") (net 1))
 (segment (start 147 108.5) (end 147 105.955) (width 0.2) (layer "F.Cu") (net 1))
 (segment (start 149.90675 100.5755) (end 149.85775 100.5265) (width 0.2) (layer "F.Cu") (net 1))
 (segment (start 136.935 103.815) (end 137.25 103.5) (width 0.2) (layer "F.Cu") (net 1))
 (segment (start 138.205 103.795) (end 138.5 103.5) (width 0.2) (layer "F.Cu") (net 1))
 (segment (start 147 105.955) (end 147.095 105.86) (width 0.2) (layer "F.Cu") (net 1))
 (segment (start 138.205 105.86) (end 138.205 103.795) (width 0.2) (layer "F.Cu") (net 1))
 (segment (start 146.99775 100.5265) (end 146.35675 101.1675) (width 0.2) (layer "F.Cu") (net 1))
 (segment (start 144.25 106.165) (end 144.555 105.86) (width 0.2) (layer "F.Cu") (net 1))
 (segment (start 146.51675 101.3275) (end 146.35675 101.1675) (width 0.2) (layer "F.Cu") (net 1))
 (segment (start 149.90675 101.3275) (end 149.90675 100.5755) (width 0.2) (layer "F.Cu") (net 1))
 (segment (start 139.475 104.025) (end 139.75 103.75) (width 0.2) (layer "F.Cu") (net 1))
 (segment (start 147.90675 101.3275) (end 146.51675 101.3275) (width 0.2) (layer "F.Cu") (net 1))
 (segment (start 136.935 105.86) (end 136.935 103.815) (width 0.2) (layer "F.Cu") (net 1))
 (segment (start 145.5 108.5) (end 145.5 106.185) (width 0.2) (layer "F.Cu") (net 1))
 (segment (start 139.475 105.86) (end 139.475 104.025) (width 0.2) (layer "F.Cu") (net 1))
 (segment (start 149.85775 100.5265) (end 146.99775 100.5265) (width 0.2) (layer "F.Cu") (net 1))
 (segment (start 154.79675 101.3275) (end 154.95675 101.1675) (width 0.2) (layer "F.Cu") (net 1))
 (via (at 147 108.5) (size 0.6) (drill 0.3) (layers "F.Cu" "B.Cu") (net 1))
 (via (at 137.25 103.5) (size 0.6) (drill 0.3) (layers "F.Cu" "B.Cu") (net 1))
 (via (at 144.25 108.25) (size 0.6) (drill 0.3) (layers "F.Cu" "B.Cu") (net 1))
 (via (at 145.5 108.5) (size 0.6) (drill 0.3) (layers "F.Cu" "B.Cu") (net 1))
 (via (at 138.5 103.5) (size 0.6) (drill 0.3) (layers "F.Cu" "B.Cu") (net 1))
 (via (at 139.75 103.75) (size 0.6) (drill 0.3) (layers "F.Cu" "B.Cu") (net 1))
 (segment (start 151.40675 102.59325) (end 151 103) (width 0.2) (layer "F.Cu") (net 4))
 (segment (start 151.40675 101.3275) (end 151.40675 102.59325) (width 0.2) (layer "F.Cu") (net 4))
 (segment (start 149.40675 102.59325) (end 149 103) (width 0.2) (layer "F.Cu") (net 4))
 (segment (start 149.40675 101.3275) (end 149.40675 102.59325) (width 0.2) (layer "F.Cu") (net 4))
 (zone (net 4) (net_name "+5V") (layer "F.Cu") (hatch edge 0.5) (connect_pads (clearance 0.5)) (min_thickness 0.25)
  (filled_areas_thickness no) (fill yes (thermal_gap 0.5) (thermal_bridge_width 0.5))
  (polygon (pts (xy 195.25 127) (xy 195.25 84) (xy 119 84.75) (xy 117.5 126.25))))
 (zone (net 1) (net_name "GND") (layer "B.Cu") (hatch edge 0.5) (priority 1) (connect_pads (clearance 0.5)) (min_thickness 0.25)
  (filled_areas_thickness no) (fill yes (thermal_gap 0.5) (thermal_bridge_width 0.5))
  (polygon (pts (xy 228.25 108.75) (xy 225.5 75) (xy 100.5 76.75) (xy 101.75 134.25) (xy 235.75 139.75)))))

